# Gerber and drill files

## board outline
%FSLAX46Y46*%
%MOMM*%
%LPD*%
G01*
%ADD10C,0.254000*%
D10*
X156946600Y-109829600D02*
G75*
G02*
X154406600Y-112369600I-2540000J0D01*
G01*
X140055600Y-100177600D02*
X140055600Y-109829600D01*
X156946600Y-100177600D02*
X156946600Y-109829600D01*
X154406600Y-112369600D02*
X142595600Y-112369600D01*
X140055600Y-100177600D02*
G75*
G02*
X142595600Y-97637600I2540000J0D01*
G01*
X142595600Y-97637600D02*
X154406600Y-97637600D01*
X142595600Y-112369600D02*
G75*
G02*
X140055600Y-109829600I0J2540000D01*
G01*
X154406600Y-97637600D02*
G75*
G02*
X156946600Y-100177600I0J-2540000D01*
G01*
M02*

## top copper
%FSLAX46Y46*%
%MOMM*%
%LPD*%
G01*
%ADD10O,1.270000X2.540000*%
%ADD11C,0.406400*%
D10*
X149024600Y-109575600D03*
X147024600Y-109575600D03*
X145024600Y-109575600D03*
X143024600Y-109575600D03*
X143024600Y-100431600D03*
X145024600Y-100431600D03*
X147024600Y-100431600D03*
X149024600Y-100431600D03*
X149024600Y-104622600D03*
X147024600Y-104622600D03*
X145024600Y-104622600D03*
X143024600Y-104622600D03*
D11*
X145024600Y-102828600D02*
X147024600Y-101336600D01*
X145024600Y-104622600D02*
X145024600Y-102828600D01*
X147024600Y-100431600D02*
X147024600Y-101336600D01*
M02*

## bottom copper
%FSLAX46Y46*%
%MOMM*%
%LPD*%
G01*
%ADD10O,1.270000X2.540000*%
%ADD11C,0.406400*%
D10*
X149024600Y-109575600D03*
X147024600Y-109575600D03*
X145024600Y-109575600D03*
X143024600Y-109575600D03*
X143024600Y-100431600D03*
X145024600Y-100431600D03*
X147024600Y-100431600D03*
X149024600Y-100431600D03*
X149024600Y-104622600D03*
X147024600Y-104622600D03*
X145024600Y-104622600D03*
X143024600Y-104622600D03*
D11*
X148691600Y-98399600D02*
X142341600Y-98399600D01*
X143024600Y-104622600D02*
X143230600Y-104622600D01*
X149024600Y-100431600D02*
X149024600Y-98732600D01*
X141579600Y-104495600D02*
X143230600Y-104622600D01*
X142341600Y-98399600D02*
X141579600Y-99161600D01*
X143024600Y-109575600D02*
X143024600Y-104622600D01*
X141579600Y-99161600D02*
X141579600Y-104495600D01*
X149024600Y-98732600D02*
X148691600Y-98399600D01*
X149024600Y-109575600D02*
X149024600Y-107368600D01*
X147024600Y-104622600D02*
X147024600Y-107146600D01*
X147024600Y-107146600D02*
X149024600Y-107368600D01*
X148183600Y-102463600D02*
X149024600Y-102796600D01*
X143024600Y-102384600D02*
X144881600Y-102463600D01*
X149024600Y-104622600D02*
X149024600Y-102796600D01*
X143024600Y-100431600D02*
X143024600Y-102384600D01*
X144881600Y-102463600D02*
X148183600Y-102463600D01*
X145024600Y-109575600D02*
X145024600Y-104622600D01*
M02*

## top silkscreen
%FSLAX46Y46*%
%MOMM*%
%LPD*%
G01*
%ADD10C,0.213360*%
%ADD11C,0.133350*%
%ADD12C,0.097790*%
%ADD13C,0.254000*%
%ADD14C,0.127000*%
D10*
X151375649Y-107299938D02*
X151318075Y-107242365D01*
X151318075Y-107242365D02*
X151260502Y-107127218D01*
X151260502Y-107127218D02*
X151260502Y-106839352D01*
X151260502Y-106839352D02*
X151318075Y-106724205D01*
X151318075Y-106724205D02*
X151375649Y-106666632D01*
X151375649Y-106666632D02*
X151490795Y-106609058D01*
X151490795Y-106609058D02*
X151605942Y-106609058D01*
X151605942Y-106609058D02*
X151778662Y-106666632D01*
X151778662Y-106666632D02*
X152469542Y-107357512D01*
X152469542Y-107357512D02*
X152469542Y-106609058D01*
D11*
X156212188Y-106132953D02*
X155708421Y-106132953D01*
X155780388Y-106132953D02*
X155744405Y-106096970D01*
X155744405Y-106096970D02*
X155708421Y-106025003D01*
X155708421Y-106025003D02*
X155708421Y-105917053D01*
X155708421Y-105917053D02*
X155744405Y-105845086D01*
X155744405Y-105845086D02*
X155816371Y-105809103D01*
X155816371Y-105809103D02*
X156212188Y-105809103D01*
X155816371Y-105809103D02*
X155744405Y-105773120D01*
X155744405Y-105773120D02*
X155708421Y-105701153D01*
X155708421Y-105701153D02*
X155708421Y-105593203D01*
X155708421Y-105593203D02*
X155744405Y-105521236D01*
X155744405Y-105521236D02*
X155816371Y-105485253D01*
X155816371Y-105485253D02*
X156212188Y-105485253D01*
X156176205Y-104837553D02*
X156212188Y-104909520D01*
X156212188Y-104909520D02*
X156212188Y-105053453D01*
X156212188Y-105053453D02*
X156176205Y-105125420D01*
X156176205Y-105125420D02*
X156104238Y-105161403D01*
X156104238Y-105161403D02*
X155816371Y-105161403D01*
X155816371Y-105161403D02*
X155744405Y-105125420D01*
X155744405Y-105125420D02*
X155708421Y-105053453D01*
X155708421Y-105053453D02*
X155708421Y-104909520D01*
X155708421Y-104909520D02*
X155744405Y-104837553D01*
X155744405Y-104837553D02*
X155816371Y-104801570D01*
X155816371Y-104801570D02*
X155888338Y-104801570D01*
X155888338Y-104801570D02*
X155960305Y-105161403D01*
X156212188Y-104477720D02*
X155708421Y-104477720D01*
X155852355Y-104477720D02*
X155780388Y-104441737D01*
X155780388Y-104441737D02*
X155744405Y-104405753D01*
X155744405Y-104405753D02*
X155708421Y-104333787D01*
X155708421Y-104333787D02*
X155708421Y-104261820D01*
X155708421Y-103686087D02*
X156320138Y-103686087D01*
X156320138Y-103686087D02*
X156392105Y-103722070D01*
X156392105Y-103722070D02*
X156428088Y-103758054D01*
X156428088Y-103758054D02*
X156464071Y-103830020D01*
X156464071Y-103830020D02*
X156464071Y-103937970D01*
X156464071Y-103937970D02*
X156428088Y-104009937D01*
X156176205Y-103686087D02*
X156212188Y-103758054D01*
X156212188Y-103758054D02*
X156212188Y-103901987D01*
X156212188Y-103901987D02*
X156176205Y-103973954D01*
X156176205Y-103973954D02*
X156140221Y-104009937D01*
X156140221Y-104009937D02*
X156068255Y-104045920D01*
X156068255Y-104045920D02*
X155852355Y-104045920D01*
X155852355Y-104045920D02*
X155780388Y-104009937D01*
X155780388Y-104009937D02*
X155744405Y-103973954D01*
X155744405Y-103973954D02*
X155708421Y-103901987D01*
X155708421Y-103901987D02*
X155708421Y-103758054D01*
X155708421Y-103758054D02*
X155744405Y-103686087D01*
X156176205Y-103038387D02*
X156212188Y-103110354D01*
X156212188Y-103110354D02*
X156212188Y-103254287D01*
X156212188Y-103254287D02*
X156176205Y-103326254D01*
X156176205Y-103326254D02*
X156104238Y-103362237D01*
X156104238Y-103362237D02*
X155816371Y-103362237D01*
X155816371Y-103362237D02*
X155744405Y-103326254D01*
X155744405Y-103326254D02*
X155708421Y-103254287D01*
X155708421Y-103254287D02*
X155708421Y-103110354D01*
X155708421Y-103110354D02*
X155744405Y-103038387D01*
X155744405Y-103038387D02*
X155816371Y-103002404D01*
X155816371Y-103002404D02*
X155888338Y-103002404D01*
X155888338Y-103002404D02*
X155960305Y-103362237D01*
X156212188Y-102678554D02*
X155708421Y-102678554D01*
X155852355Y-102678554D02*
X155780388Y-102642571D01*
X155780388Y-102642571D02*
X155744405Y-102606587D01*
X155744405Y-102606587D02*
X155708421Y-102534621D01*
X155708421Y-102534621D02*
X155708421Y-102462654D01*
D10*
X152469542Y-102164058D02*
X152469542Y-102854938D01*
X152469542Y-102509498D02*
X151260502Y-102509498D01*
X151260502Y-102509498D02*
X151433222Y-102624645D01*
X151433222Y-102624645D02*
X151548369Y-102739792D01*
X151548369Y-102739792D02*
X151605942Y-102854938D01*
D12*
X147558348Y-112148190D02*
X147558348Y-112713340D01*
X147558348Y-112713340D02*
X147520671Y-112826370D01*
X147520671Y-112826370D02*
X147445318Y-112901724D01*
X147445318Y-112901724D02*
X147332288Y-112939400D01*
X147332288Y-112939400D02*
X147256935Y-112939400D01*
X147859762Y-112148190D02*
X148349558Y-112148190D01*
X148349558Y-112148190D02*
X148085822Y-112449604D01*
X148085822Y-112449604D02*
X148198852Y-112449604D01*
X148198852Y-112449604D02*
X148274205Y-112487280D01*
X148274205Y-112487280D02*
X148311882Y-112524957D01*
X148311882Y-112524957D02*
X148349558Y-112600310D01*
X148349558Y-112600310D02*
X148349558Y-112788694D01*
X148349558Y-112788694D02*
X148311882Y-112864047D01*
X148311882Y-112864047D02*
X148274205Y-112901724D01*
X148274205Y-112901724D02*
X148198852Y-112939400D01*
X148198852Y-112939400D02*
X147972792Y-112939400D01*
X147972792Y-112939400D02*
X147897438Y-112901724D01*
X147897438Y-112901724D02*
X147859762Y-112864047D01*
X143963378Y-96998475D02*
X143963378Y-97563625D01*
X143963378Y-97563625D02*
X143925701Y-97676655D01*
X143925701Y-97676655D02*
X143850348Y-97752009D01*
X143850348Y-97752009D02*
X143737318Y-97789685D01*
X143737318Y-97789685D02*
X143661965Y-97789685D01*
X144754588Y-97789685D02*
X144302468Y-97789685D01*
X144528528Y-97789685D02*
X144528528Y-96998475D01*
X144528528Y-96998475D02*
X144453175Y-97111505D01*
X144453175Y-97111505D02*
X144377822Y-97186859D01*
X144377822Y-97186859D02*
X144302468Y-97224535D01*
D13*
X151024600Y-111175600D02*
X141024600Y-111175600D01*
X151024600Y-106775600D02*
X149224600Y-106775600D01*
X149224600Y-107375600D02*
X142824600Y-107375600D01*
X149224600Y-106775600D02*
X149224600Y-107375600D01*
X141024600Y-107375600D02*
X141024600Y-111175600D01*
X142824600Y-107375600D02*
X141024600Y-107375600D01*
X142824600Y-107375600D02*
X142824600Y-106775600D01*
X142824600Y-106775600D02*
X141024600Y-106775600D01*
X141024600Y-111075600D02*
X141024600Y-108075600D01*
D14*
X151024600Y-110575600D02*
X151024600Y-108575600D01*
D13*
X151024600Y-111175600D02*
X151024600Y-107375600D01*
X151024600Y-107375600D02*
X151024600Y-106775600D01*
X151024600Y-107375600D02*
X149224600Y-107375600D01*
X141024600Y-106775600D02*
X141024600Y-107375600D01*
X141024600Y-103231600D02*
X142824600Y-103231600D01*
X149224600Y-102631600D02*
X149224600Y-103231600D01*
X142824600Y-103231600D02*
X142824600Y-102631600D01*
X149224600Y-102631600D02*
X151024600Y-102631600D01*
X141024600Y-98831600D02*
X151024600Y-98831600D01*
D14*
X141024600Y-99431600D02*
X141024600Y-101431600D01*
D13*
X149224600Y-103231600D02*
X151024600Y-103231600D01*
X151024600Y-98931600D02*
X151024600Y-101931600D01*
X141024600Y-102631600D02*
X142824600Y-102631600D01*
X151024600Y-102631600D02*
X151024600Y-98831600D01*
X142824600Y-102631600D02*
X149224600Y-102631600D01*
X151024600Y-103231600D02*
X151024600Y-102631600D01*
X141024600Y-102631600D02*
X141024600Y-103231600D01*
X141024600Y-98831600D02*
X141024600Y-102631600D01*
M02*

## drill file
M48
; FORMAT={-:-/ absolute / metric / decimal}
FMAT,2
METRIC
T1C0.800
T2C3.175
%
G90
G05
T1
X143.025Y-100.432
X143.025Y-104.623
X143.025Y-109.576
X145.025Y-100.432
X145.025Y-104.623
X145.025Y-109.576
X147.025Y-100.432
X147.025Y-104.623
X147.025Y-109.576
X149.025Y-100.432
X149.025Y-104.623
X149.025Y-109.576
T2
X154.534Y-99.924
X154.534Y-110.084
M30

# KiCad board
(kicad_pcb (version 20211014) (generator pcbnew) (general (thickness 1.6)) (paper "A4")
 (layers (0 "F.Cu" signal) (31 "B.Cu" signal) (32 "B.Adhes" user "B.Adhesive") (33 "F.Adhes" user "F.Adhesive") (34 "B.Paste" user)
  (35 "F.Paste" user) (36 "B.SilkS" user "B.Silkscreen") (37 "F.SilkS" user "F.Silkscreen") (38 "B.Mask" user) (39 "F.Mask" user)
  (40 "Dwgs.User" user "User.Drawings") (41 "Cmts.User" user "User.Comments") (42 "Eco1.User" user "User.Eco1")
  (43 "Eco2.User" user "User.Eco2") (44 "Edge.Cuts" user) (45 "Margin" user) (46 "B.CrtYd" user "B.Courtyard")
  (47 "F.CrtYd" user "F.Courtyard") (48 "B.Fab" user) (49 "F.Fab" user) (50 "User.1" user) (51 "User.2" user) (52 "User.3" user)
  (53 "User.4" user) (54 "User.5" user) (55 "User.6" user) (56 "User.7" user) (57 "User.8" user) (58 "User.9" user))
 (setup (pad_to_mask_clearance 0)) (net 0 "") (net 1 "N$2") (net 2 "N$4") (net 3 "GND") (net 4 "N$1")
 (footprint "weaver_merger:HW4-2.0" (layer "F.Cu") (at 146.0246 109.5756 180)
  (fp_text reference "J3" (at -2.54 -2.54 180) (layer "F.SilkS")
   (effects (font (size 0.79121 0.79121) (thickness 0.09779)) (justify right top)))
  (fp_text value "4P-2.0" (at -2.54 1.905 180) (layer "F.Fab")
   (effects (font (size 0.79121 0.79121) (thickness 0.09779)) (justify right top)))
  (fp_line (start -5 -1.6) (end 5 -1.6) (layer "F.SilkS") (width 0.254))
  (fp_line (start -5 2.8) (end -3.2 2.8) (layer "F.SilkS") (width 0.254))
  (fp_line (start -3.2 2.2) (end 3.2 2.2) (layer "F.SilkS") (width 0.254))
  (fp_line (start -3.2 2.8) (end -3.2 2.2) (layer "F.SilkS") (width 0.254))
  (fp_line (start 5 2.2) (end 5 -1.6) (layer "F.SilkS") (width 0.254))
  (fp_line (start 3.2 2.2) (end 5 2.2) (layer "F.SilkS") (width 0.254))
  (fp_line (start 3.2 2.2) (end 3.2 2.8) (layer "F.SilkS") (width 0.254))
  (fp_line (start 3.2 2.8) (end 5 2.8) (layer "F.SilkS") (width 0.254))
  (fp_line (start 5 -1.5) (end 5 1.5) (layer "F.SilkS") (width 0.254))
  (fp_line (start -5 -1) (end -5 1) (layer "F.SilkS") (width 0.127))
  (fp_line (start -5 -1.6) (end -5 2.2) (layer "F.SilkS") (width 0.254))
  (fp_line (start -5 2.2) (end -5 2.8) (layer "F.SilkS") (width 0.254))
  (fp_line (start -5 2.2) (end -3.2 2.2) (layer "F.SilkS") (width 0.254))
  (fp_line (start 5 2.8) (end 5 2.2) (layer "F.SilkS") (width 0.254))
  (pad "1" thru_hole oval (at -3 0 270) (size 2.54 1.27) (drill 0.8) (layers *.Cu *.Mask) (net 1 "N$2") (solder_mask_margin 0.1016))
  (pad "2" thru_hole oval (at -1 0 270) (size 2.54 1.27) (drill 0.8) (layers *.Cu *.Mask) (solder_mask_margin 0.1016))
  (pad "3" thru_hole oval (at 1 0 270) (size 2.54 1.27) (drill 0.8) (layers *.Cu *.Mask) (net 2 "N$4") (solder_mask_margin 0.1016))
  (pad "4" thru_hole oval (at 3 0 270) (size 2.54 1.27) (drill 0.8) (layers *.Cu *.Mask) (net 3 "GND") (solder_mask_margin 0.1016)))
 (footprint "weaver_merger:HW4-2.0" (layer "F.Cu") (at 146.0246 100.4316)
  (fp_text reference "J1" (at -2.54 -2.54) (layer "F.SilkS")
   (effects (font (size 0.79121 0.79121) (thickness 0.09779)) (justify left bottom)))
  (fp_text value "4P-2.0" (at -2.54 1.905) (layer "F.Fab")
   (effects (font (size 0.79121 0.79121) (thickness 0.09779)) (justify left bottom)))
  (fp_line (start -5 2.8) (end -3.2 2.8) (layer "F.SilkS") (width 0.254))
  (fp_line (start 3.2 2.2) (end 3.2 2.8) (layer "F.SilkS") (width 0.254))
  (fp_line (start -3.2 2.8) (end -3.2 2.2) (layer "F.SilkS") (width 0.254))
  (fp_line (start 3.2 2.2) (end 5 2.2) (layer "F.SilkS") (width 0.254))
  (fp_line (start -5 -1.6) (end 5 -1.6) (layer "F.SilkS") (width 0.254))
  (fp_line (start -5 -1) (end -5 1) (layer "F.SilkS") (width 0.127))
  (fp_line (start 3.2 2.8) (end 5 2.8) (layer "F.SilkS") (width 0.254))
  (fp_line (start 5 -1.5) (end 5 1.5) (layer "F.SilkS") (width 0.254))
  (fp_line (start -5 2.2) (end -3.2 2.2) (layer "F.SilkS") (width 0.254))
  (fp_line (start 5 2.2) (end 5 -1.6) (layer "F.SilkS") (width 0.254))
  (fp_line (start -3.2 2.2) (end 3.2 2.2) (layer "F.SilkS") (width 0.254))
  (fp_line (start 5 2.8) (end 5 2.2) (layer "F.SilkS") (width 0.254))
  (fp_line (start -5 2.2) (end -5 2.8) (layer "F.SilkS") (width 0.254))
  (fp_line (start -5 -1.6) (end -5 2.2) (layer "F.SilkS") (width 0.254))
  (pad "1" thru_hole oval (at -3 0 90) (size 2.54 1.27) (drill 0.8) (layers *.Cu *.Mask) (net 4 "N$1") (solder_mask_margin 0.1016))
  (pad "2" thru_hole oval (at -1 0 90) (size 2.54 1.27) (drill 0.8) (layers *.Cu *.Mask) (solder_mask_margin 0.1016))
  (pad "3" thru_hole oval (at 1 0 90) (size 2.54 1.27) (drill 0.8) (layers *.Cu *.Mask) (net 2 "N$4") (solder_mask_margin 0.1016))
  (pad "4" thru_hole oval (at 3 0 90) (size 2.54 1.27) (drill 0.8) (layers *.Cu *.Mask) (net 3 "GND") (solder_mask_margin 0.1016)))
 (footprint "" (layer "F.Cu") (at 154.5336 110.0836)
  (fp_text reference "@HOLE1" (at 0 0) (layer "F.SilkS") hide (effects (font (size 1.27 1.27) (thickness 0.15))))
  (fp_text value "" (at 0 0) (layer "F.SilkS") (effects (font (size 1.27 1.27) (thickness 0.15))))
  (pad "" np_thru_hole circle (at 0 0) (size 3.175 3.175) (drill 3.175) (layers *.Cu *.Mask)))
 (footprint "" (layer "F.Cu") (at 154.5336 99.9236)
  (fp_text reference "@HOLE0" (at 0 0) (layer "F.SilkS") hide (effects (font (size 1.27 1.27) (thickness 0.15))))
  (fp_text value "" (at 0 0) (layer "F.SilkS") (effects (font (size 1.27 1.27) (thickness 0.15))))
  (pad "" np_thru_hole circle (at 0 0) (size 3.175 3.175) (drill 3.175) (layers *.Cu *.Mask)))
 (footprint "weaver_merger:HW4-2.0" (layer "B.Cu") (at 146.0246 104.6226 180)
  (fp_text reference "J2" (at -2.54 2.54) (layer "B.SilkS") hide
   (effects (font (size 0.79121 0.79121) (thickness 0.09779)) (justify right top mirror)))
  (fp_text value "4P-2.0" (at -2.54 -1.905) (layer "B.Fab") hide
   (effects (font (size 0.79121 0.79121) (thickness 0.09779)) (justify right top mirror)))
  (pad "1" thru_hole oval (at -3 0 90) (size 2.54 1.27) (drill 0.8) (layers *.Cu *.Mask) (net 4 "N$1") (solder_mask_margin 0.1016))
  (pad "2" thru_hole oval (at -1 0 90) (size 2.54 1.27) (drill 0.8) (layers *.Cu *.Mask) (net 1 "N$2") (solder_mask_margin 0.1016))
  (pad "3" thru_hole oval (at 1 0 90) (size 2.54 1.27) (drill 0.8) (layers *.Cu *.Mask) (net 2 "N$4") (solder_mask_margin 0.1016))
  (pad "4" thru_hole oval (at 3 0 90) (size 2.54 1.27) (drill 0.8) (layers *.Cu *.Mask) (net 3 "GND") (solder_mask_margin 0.1016)))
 (gr_arc (start 156.9466 109.8296) (mid 156.202651 111.625651) (end 154.4066 112.3696) (layer "Edge.Cuts") (width 0.254))
 (gr_line (start 140.0556 100.1776) (end 140.0556 109.8296) (layer "Edge.Cuts") (width 0.254))
 (gr_line (start 156.9466 100.1776) (end 156.9466 109.8296) (layer "Edge.Cuts") (width 0.254))
 (gr_line (start 154.4066 112.3696) (end 142.5956 112.3696) (layer "Edge.Cuts") (width 0.254))
 (gr_arc (start 140.0556 100.1776) (mid 140.799549 98.381549) (end 142.5956 97.6376) (layer "Edge.Cuts") (width 0.254))
 (gr_line (start 142.5956 97.6376) (end 154.4066 97.6376) (layer "Edge.Cuts") (width 0.254))
 (gr_arc (start 142.5956 112.3696) (mid 140.799549 111.625651) (end 140.0556 109.8296) (layer "Edge.Cuts") (width 0.254))
 (gr_arc (start 154.4066 97.6376) (mid 156.202651 98.381549) (end 156.9466 100.1776) (layer "Edge.Cuts") (width 0.254))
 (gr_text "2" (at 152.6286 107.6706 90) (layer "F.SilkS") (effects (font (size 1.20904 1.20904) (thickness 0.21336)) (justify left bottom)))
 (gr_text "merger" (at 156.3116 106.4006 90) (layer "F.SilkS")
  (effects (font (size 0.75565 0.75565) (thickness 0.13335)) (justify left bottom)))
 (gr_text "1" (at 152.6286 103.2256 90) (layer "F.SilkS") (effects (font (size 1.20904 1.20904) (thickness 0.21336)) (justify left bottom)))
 (segment (start 148.6916 98.3996) (end 142.3416 98.3996) (width 0.4064) (layer "B.Cu") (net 3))
 (segment (start 143.0246 104.6226) (end 143.2306 104.6226) (width 0.4064) (layer "B.Cu") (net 3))
 (segment (start 149.0246 100.4316) (end 149.0246 98.7326) (width 0.4064) (layer "B.Cu") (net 3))
 (segment (start 141.5796 104.4956) (end 143.2306 104.6226) (width 0.4064) (layer "B.Cu") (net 3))
 (segment (start 142.3416 98.3996) (end 141.5796 99.1616) (width 0.4064) (layer "B.Cu") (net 3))
 (segment (start 143.0246 109.5756) (end 143.0246 104.6226) (width 0.4064) (layer "B.Cu") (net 3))
 (segment (start 141.5796 99.1616) (end 141.5796 104.4956) (width 0.4064) (layer "B.Cu") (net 3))
 (segment (start 149.0246 98.7326) (end 148.6916 98.3996) (width 0.4064) (layer "B.Cu") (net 3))
 (segment (start 149.0246 109.5756) (end 149.0246 107.3686) (width 0.4064) (layer "B.Cu") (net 1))
 (segment (start 147.0246 104.6226) (end 147.0246 107.1466) (width 0.4064) (layer "B.Cu") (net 1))
 (segment (start 147.0246 107.1466) (end 149.0246 107.3686) (width 0.4064) (layer "B.Cu") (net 1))
 (segment (start 148.1836 102.4636) (end 149.0246 102.7966) (width 0.4064) (layer "B.Cu") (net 4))
 (segment (start 143.0246 102.3846) (end 144.8816 102.4636) (width 0.4064) (layer "B.Cu") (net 4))
 (segment (start 149.0246 104.6226) (end 149.0246 102.7966) (width 0.4064) (layer "B.Cu") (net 4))
 (segment (start 143.0246 100.4316) (end 143.0246 102.3846) (width 0.4064) (layer "B.Cu") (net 4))
 (segment (start 144.8816 102.4636) (end 148.1836 102.4636) (width 0.4064) (layer "B.Cu") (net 4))
 (segment (start 145.0246 102.8286) (end 147.0246 101.3366) (width 0.4064) (layer "F.Cu") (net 2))
 (segment (start 145.0246 104.6226) (end 145.0246 102.8286) (width 0.4064) (layer "F.Cu") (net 2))
 (segment (start 147.0246 100.4316) (end 147.0246 101.3366) (width 0.4064) (layer "F.Cu") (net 2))
 (segment (start 145.0246 109.5756) (end 145.0246 104.6226) (width 0.4064) (layer "B.Cu") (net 2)))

